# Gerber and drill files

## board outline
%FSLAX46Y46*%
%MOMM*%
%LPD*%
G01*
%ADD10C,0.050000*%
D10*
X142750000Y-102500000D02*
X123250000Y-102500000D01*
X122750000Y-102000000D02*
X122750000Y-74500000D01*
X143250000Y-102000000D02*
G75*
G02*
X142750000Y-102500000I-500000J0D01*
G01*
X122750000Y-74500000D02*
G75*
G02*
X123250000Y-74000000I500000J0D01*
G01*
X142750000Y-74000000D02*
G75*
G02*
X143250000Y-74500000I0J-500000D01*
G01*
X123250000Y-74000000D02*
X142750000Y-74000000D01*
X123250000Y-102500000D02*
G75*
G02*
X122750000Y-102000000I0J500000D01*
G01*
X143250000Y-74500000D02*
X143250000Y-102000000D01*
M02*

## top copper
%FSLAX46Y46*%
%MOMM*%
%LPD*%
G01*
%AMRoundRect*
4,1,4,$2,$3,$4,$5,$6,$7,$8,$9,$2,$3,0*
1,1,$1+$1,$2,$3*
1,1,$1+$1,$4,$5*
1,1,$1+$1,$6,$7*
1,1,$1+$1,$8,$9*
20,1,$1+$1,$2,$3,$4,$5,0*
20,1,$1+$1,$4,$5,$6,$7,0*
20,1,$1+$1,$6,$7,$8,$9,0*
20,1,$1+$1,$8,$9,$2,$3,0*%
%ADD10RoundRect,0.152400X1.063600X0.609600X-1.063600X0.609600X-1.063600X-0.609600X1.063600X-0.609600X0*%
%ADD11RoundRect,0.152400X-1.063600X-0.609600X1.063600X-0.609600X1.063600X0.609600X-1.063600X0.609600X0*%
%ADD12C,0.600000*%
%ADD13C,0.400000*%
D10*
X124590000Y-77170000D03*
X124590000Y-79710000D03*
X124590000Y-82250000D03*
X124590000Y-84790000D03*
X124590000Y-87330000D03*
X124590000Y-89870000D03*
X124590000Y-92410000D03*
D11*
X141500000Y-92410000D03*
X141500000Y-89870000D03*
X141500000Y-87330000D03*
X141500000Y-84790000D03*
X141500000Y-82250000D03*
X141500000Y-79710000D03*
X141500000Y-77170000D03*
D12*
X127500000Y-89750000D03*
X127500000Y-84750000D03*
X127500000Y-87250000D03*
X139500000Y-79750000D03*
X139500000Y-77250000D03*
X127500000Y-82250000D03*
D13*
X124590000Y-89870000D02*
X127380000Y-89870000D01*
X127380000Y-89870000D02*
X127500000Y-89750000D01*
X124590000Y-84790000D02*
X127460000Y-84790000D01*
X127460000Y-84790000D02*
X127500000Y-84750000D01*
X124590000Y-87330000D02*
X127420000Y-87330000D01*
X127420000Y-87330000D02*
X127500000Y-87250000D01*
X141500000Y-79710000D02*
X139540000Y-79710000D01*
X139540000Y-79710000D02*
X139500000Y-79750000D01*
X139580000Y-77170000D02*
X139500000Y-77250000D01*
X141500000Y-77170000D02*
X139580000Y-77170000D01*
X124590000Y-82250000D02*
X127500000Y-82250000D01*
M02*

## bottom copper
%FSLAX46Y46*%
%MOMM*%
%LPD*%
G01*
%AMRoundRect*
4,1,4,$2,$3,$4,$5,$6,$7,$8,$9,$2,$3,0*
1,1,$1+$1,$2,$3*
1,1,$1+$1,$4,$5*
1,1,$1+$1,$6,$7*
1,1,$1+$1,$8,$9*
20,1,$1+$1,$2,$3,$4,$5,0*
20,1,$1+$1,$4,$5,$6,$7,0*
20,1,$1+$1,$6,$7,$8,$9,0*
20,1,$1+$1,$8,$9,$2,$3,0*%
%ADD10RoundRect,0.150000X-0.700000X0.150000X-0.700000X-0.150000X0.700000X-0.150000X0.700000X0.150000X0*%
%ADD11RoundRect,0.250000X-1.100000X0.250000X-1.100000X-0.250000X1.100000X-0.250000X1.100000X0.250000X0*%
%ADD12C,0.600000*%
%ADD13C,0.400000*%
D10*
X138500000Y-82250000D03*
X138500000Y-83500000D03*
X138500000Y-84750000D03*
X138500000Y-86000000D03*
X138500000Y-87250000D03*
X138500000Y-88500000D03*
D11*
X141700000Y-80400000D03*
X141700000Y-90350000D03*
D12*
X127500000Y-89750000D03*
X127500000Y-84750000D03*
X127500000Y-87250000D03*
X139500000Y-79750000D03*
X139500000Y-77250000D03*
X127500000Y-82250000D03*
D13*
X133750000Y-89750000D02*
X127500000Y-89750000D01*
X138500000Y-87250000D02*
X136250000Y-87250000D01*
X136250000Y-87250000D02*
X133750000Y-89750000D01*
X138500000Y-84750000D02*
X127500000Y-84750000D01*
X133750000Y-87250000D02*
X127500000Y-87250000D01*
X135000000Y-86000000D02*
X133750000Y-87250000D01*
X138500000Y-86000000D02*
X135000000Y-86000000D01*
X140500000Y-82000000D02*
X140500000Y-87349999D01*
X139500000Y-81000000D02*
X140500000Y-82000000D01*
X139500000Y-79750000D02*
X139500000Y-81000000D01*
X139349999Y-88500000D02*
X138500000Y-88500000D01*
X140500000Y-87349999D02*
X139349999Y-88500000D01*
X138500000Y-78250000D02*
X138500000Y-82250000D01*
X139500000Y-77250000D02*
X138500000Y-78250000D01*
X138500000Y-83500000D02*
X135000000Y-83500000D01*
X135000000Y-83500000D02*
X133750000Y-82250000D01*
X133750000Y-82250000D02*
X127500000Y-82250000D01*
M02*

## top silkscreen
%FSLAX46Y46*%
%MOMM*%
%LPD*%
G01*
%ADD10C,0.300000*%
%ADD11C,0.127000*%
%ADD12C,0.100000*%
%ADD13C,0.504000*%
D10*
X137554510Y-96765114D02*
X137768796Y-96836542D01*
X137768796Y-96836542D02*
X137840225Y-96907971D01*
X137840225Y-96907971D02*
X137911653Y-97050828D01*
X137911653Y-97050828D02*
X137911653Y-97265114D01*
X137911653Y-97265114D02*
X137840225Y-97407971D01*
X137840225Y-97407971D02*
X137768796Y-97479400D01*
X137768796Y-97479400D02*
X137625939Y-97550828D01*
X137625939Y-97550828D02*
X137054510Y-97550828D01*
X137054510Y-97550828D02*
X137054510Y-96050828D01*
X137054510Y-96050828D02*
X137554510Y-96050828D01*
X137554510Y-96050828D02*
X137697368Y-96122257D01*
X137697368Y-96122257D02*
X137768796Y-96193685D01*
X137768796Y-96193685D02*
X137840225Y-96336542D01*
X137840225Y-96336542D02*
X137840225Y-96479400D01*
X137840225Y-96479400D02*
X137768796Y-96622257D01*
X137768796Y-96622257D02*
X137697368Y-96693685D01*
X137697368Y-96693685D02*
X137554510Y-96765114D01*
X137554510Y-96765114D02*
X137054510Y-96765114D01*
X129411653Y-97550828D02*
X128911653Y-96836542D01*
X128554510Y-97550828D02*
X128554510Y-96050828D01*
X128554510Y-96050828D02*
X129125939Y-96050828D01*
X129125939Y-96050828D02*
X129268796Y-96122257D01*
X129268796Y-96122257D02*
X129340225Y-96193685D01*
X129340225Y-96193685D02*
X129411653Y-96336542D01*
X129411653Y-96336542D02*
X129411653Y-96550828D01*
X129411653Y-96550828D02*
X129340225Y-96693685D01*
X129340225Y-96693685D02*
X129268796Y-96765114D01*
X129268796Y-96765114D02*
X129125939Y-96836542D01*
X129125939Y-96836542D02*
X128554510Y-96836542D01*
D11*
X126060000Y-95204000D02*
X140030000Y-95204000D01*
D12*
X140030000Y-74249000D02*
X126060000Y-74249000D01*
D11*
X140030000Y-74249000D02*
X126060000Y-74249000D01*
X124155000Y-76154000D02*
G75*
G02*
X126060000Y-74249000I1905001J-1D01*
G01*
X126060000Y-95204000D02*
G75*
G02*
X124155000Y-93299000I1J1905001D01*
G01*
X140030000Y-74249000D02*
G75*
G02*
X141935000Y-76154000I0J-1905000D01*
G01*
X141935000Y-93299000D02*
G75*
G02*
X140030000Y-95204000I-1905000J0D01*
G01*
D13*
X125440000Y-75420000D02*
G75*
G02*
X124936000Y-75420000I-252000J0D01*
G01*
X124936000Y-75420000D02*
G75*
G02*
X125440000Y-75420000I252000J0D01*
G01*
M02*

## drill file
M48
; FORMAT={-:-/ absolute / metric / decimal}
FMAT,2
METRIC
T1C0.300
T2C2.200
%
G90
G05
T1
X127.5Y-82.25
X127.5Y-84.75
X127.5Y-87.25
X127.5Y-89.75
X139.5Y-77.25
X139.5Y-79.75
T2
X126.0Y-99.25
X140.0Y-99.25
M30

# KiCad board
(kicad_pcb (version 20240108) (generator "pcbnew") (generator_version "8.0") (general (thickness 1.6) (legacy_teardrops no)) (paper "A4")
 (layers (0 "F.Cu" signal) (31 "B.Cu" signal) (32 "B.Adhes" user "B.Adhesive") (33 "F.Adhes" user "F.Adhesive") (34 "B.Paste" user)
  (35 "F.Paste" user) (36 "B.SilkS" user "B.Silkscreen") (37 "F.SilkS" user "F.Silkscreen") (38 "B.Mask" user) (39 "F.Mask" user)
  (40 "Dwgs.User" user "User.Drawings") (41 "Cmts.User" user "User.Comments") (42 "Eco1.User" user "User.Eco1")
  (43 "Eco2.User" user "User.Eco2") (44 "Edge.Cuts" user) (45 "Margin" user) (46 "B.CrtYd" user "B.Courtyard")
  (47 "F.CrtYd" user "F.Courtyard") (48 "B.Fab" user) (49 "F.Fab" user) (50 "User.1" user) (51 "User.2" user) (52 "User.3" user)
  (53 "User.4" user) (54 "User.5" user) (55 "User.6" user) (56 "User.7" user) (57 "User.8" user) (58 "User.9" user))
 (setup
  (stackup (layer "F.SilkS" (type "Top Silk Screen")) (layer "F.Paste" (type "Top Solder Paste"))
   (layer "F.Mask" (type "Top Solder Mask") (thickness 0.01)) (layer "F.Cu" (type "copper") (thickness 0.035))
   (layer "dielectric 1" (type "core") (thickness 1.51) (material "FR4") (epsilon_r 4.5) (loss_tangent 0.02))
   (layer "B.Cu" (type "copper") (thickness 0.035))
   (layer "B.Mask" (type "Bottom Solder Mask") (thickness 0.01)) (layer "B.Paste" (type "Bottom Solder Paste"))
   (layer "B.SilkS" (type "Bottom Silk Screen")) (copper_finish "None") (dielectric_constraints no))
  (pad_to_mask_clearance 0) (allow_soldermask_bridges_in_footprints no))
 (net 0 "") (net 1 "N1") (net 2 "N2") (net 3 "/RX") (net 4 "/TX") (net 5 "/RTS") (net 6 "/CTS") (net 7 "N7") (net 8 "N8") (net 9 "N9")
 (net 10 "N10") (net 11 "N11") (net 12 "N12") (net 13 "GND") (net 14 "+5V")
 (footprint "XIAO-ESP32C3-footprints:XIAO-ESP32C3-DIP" (layer "F.Cu") (at 133.165 84.79)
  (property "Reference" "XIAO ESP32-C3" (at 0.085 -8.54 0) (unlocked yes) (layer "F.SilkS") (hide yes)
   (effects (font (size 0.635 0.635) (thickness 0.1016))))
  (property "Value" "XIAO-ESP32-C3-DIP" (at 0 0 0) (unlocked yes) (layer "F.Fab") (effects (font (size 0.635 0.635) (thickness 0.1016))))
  (fp_line (start -7.105 10.414) (end 6.865 10.414) (stroke (width 0.127) (type solid)) (layer "F.SilkS"))
  (fp_line (start 6.865 -10.541) (end -7.105 -10.541) (stroke (width 0.1) (type solid)) (layer "F.SilkS"))
  (fp_line (start 6.865 -10.541) (end -7.105 -10.541) (stroke (width 0.127) (type solid)) (layer "F.SilkS"))
  (fp_arc (start -9.01 -8.636) (mid -8.452038 -9.983038) (end -7.105 -10.541) (stroke (width 0.127) (type solid)) (layer "F.SilkS"))
  (fp_arc (start -7.105 10.414) (mid -8.452038 9.856038) (end -9.01 8.509) (stroke (width 0.127) (type solid)) (layer "F.SilkS"))
  (fp_arc (start 6.865 -10.541) (mid 8.212038 -9.983038) (end 8.77 -8.636) (stroke (width 0.127) (type solid)) (layer "F.SilkS"))
  (fp_arc (start 8.77 8.509) (mid 8.212038 9.856038) (end 6.865 10.414) (stroke (width 0.127) (type solid)) (layer "F.SilkS"))
  (fp_circle (center -7.977 -9.37) (end -7.977 -9.624) (stroke (width 0.5) (type solid)) (fill solid) (layer "F.SilkS"))
  (pad "1" smd roundrect (at -8.575 -7.62 180) (size 2.432 1.524) (layers "F.Cu" "F.Mask") (roundrect_rratio 0.1) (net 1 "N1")
   (thermal_bridge_angle 45))
  (pad "2" smd roundrect (at -8.575 -5.08 180) (size 2.432 1.524) (layers "F.Cu" "F.Mask") (roundrect_rratio 0.1) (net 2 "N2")
   (thermal_bridge_angle 45))
  (pad "3" smd roundrect (at -8.575 -2.54 180) (size 2.432 1.524) (layers "F.Cu" "F.Mask") (roundrect_rratio 0.1) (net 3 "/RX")
   (thermal_bridge_angle 45))
  (pad "4" smd roundrect (at -8.575 0 180) (size 2.432 1.524) (layers "F.Cu" "F.Mask") (roundrect_rratio 0.1) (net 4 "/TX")
   (thermal_bridge_angle 45))
  (pad "5" smd roundrect (at -8.575 2.54 180) (size 2.432 1.524) (layers "F.Cu" "F.Mask") (roundrect_rratio 0.1) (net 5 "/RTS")
   (thermal_bridge_angle 45))
  (pad "6" smd roundrect (at -8.575 5.08 180) (size 2.432 1.524) (layers "F.Cu" "F.Mask") (roundrect_rratio 0.1) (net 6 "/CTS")
   (thermal_bridge_angle 45))
  (pad "7" smd roundrect (at -8.575 7.62 180) (size 2.432 1.524) (layers "F.Cu" "F.Mask") (roundrect_rratio 0.1) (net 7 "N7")
   (thermal_bridge_angle 45))
  (pad "8" smd roundrect (at 8.335 7.62) (size 2.432 1.524) (layers "F.Cu" "F.Mask") (roundrect_rratio 0.1) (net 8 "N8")
   (thermal_bridge_angle 45))
  (pad "9" smd roundrect (at 8.335 5.08) (size 2.432 1.524) (layers "F.Cu" "F.Mask") (roundrect_rratio 0.1) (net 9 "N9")
   (thermal_bridge_angle 45))
  (pad "10" smd roundrect (at 8.335 2.54) (size 2.432 1.524) (layers "F.Cu" "F.Mask") (roundrect_rratio 0.1) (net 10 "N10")
   (thermal_bridge_angle 45))
  (pad "11" smd roundrect (at 8.335 0) (size 2.432 1.524) (layers "F.Cu" "F.Mask") (roundrect_rratio 0.1) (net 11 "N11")
   (thermal_bridge_angle 45))
  (pad "12" smd roundrect (at 8.335 -2.54) (size 2.432 1.524) (layers "F.Cu" "F.Mask") (roundrect_rratio 0.1) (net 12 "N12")
   (thermal_bridge_angle 45))
  (pad "13" smd roundrect (at 8.335 -5.08) (size 2.432 1.524) (layers "F.Cu" "F.Mask") (roundrect_rratio 0.1) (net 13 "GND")
   (thermal_bridge_angle 45))
  (pad "14" smd roundrect (at 8.335 -7.62) (size 2.432 1.524) (layers "F.Cu" "F.Mask") (roundrect_rratio 0.1) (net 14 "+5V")
   (thermal_bridge_angle 45)))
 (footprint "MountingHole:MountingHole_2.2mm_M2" (layer "F.Cu") (at 140 99.25)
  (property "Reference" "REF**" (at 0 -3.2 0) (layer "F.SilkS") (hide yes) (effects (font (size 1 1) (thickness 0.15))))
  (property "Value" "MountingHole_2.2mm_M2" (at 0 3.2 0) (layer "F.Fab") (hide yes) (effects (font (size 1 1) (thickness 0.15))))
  (pad "" np_thru_hole circle (at 0 0) (size 2.2 2.2) (drill 2.2) (layers "*.Cu" "*.Mask")))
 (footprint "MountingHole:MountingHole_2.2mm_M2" (layer "F.Cu") (at 126 99.25)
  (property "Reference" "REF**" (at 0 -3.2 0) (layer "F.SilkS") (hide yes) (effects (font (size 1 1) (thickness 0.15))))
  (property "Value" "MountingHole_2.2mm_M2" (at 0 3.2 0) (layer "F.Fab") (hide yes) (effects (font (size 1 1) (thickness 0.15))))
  (pad "" np_thru_hole circle (at 0 0) (size 2.2 2.2) (drill 2.2) (layers "*.Cu" "*.Mask")))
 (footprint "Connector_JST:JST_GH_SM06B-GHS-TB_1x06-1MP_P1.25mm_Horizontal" (layer "B.Cu") (at 140.35 85.375 -90)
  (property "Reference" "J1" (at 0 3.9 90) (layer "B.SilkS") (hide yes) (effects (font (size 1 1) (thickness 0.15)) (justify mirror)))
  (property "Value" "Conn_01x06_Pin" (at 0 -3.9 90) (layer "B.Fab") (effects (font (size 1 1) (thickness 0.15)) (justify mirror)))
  (pad "1" smd roundrect (at -3.125 1.85 270) (size 0.6 1.7) (layers "B.Cu" "B.Paste" "B.Mask") (roundrect_rratio 0.25) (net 14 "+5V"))
  (pad "2" smd roundrect (at -1.875 1.85 270) (size 0.6 1.7) (layers "B.Cu" "B.Paste" "B.Mask") (roundrect_rratio 0.25) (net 3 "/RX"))
  (pad "3" smd roundrect (at -0.625 1.85 270) (size 0.6 1.7) (layers "B.Cu" "B.Paste" "B.Mask") (roundrect_rratio 0.25) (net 4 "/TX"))
  (pad "4" smd roundrect (at 0.625 1.85 270) (size 0.6 1.7) (layers "B.Cu" "B.Paste" "B.Mask") (roundrect_rratio 0.25) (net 5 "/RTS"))
  (pad "5" smd roundrect (at 1.875 1.85 270) (size 0.6 1.7) (layers "B.Cu" "B.Paste" "B.Mask") (roundrect_rratio 0.25) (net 6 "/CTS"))
  (pad "6" smd roundrect (at 3.125 1.85 270) (size 0.6 1.7) (layers "B.Cu" "B.Paste" "B.Mask") (roundrect_rratio 0.25) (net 13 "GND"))
  (pad "MP" smd roundrect (at -4.975 -1.35 270) (size 1 2.7) (layers "B.Cu" "B.Paste" "B.Mask") (roundrect_rratio 0.25))
  (pad "MP" smd roundrect (at 4.975 -1.35 270) (size 1 2.7) (layers "B.Cu" "B.Paste" "B.Mask") (roundrect_rratio 0.25)))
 (gr_line (start 142.75 102.5) (end 123.25 102.5) (stroke (width 0.05) (type default)) (layer "Edge.Cuts"))
 (gr_line (start 122.75 102) (end 122.75 74.5) (stroke (width 0.05) (type default)) (layer "Edge.Cuts"))
 (gr_arc (start 143.25 102) (mid 143.103553 102.353553) (end 142.75 102.5) (stroke (width 0.05) (type default)) (layer "Edge.Cuts"))
 (gr_arc (start 122.75 74.5) (mid 122.896447 74.146447) (end 123.25 74) (stroke (width 0.05) (type default)) (layer "Edge.Cuts"))
 (gr_arc (start 142.75 74) (mid 143.103553 74.146447) (end 143.25 74.5) (stroke (width 0.05) (type default)) (layer "Edge.Cuts"))
 (gr_line (start 123.25 74) (end 142.75 74) (stroke (width 0.05) (type default)) (layer "Edge.Cuts"))
 (gr_arc (start 123.25 102.5) (mid 122.896447 102.353553) (end 122.75 102) (stroke (width 0.05) (type default)) (layer "Edge.Cuts"))
 (gr_line (start 143.25 74.5) (end 143.25 102) (stroke (width 0.05) (type default)) (layer "Edge.Cuts"))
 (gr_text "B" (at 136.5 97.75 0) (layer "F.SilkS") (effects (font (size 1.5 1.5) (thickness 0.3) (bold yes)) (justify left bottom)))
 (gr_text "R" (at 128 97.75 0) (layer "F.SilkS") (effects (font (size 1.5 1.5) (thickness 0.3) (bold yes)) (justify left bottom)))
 (segment (start 124.59 89.87) (end 127.38 89.87) (width 0.4) (layer "F.Cu") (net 6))
 (segment (start 127.38 89.87) (end 127.5 89.75) (width 0.4) (layer "F.Cu") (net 6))
 (via (at 127.5 89.75) (size 0.6) (drill 0.3) (layers "F.Cu" "B.Cu") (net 6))
 (segment (start 133.75 89.75) (end 127.5 89.75) (width 0.4) (layer "B.Cu") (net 6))
 (segment (start 138.5 87.25) (end 136.25 87.25) (width 0.4) (layer "B.Cu") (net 6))
 (segment (start 136.25 87.25) (end 133.75 89.75) (width 0.4) (layer "B.Cu") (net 6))
 (segment (start 124.59 84.79) (end 127.46 84.79) (width 0.4) (layer "F.Cu") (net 4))
 (segment (start 127.46 84.79) (end 127.5 84.75) (width 0.4) (layer "F.Cu") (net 4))
 (via (at 127.5 84.75) (size 0.6) (drill 0.3) (layers "F.Cu" "B.Cu") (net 4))
 (segment (start 138.5 84.75) (end 127.5 84.75) (width 0.4) (layer "B.Cu") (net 4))
 (segment (start 124.59 87.33) (end 127.42 87.33) (width 0.4) (layer "F.Cu") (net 5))
 (segment (start 127.42 87.33) (end 127.5 87.25) (width 0.4) (layer "F.Cu") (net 5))
 (via (at 127.5 87.25) (size 0.6) (drill 0.3) (layers "F.Cu" "B.Cu") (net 5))
 (segment (start 133.75 87.25) (end 127.5 87.25) (width 0.4) (layer "B.Cu") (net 5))
 (segment (start 135 86) (end 133.75 87.25) (width 0.4) (layer "B.Cu") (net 5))
 (segment (start 138.5 86) (end 135 86) (width 0.4) (layer "B.Cu") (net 5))
 (segment (start 141.5 79.71) (end 139.54 79.71) (width 0.4) (layer "F.Cu") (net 13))
 (segment (start 139.54 79.71) (end 139.5 79.75) (width 0.4) (layer "F.Cu") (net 13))
 (via (at 139.5 79.75) (size 0.6) (drill 0.3) (layers "F.Cu" "B.Cu") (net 13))
 (segment (start 140.5 82) (end 140.5 87.349999) (width 0.4) (layer "B.Cu") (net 13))
 (segment (start 139.5 81) (end 140.5 82) (width 0.4) (layer "B.Cu") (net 13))
 (segment (start 139.5 79.75) (end 139.5 81) (width 0.4) (layer "B.Cu") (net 13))
 (segment (start 139.349999 88.5) (end 138.5 88.5) (width 0.4) (layer "B.Cu") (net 13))
 (segment (start 140.5 87.349999) (end 139.349999 88.5) (width 0.4) (layer "B.Cu") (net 13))
 (segment (start 139.58 77.17) (end 139.5 77.25) (width 0.4) (layer "F.Cu") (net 14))
 (segment (start 141.5 77.17) (end 139.58 77.17) (width 0.4) (layer "F.Cu") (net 14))
 (via (at 139.5 77.25) (size 0.6) (drill 0.3) (layers "F.Cu" "B.Cu") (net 14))
 (segment (start 138.5 78.25) (end 138.5 82.25) (width 0.4) (layer "B.Cu") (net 14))
 (segment (start 139.5 77.25) (end 138.5 78.25) (width 0.4) (layer "B.Cu") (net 14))
 (segment (start 124.59 82.25) (end 127.5 82.25) (width 0.4) (layer "F.Cu") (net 3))
 (via (at 127.5 82.25) (size 0.6) (drill 0.3) (layers "F.Cu" "B.Cu") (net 3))
 (segment (start 138.5 83.5) (end 135 83.5) (width 0.4) (layer "B.Cu") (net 3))
 (segment (start 135 83.5) (end 133.75 82.25) (width 0.4) (layer "B.Cu") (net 3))
 (segment (start 133.75 82.25) (end 127.5 82.25) (width 0.4) (layer "B.Cu") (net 3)))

